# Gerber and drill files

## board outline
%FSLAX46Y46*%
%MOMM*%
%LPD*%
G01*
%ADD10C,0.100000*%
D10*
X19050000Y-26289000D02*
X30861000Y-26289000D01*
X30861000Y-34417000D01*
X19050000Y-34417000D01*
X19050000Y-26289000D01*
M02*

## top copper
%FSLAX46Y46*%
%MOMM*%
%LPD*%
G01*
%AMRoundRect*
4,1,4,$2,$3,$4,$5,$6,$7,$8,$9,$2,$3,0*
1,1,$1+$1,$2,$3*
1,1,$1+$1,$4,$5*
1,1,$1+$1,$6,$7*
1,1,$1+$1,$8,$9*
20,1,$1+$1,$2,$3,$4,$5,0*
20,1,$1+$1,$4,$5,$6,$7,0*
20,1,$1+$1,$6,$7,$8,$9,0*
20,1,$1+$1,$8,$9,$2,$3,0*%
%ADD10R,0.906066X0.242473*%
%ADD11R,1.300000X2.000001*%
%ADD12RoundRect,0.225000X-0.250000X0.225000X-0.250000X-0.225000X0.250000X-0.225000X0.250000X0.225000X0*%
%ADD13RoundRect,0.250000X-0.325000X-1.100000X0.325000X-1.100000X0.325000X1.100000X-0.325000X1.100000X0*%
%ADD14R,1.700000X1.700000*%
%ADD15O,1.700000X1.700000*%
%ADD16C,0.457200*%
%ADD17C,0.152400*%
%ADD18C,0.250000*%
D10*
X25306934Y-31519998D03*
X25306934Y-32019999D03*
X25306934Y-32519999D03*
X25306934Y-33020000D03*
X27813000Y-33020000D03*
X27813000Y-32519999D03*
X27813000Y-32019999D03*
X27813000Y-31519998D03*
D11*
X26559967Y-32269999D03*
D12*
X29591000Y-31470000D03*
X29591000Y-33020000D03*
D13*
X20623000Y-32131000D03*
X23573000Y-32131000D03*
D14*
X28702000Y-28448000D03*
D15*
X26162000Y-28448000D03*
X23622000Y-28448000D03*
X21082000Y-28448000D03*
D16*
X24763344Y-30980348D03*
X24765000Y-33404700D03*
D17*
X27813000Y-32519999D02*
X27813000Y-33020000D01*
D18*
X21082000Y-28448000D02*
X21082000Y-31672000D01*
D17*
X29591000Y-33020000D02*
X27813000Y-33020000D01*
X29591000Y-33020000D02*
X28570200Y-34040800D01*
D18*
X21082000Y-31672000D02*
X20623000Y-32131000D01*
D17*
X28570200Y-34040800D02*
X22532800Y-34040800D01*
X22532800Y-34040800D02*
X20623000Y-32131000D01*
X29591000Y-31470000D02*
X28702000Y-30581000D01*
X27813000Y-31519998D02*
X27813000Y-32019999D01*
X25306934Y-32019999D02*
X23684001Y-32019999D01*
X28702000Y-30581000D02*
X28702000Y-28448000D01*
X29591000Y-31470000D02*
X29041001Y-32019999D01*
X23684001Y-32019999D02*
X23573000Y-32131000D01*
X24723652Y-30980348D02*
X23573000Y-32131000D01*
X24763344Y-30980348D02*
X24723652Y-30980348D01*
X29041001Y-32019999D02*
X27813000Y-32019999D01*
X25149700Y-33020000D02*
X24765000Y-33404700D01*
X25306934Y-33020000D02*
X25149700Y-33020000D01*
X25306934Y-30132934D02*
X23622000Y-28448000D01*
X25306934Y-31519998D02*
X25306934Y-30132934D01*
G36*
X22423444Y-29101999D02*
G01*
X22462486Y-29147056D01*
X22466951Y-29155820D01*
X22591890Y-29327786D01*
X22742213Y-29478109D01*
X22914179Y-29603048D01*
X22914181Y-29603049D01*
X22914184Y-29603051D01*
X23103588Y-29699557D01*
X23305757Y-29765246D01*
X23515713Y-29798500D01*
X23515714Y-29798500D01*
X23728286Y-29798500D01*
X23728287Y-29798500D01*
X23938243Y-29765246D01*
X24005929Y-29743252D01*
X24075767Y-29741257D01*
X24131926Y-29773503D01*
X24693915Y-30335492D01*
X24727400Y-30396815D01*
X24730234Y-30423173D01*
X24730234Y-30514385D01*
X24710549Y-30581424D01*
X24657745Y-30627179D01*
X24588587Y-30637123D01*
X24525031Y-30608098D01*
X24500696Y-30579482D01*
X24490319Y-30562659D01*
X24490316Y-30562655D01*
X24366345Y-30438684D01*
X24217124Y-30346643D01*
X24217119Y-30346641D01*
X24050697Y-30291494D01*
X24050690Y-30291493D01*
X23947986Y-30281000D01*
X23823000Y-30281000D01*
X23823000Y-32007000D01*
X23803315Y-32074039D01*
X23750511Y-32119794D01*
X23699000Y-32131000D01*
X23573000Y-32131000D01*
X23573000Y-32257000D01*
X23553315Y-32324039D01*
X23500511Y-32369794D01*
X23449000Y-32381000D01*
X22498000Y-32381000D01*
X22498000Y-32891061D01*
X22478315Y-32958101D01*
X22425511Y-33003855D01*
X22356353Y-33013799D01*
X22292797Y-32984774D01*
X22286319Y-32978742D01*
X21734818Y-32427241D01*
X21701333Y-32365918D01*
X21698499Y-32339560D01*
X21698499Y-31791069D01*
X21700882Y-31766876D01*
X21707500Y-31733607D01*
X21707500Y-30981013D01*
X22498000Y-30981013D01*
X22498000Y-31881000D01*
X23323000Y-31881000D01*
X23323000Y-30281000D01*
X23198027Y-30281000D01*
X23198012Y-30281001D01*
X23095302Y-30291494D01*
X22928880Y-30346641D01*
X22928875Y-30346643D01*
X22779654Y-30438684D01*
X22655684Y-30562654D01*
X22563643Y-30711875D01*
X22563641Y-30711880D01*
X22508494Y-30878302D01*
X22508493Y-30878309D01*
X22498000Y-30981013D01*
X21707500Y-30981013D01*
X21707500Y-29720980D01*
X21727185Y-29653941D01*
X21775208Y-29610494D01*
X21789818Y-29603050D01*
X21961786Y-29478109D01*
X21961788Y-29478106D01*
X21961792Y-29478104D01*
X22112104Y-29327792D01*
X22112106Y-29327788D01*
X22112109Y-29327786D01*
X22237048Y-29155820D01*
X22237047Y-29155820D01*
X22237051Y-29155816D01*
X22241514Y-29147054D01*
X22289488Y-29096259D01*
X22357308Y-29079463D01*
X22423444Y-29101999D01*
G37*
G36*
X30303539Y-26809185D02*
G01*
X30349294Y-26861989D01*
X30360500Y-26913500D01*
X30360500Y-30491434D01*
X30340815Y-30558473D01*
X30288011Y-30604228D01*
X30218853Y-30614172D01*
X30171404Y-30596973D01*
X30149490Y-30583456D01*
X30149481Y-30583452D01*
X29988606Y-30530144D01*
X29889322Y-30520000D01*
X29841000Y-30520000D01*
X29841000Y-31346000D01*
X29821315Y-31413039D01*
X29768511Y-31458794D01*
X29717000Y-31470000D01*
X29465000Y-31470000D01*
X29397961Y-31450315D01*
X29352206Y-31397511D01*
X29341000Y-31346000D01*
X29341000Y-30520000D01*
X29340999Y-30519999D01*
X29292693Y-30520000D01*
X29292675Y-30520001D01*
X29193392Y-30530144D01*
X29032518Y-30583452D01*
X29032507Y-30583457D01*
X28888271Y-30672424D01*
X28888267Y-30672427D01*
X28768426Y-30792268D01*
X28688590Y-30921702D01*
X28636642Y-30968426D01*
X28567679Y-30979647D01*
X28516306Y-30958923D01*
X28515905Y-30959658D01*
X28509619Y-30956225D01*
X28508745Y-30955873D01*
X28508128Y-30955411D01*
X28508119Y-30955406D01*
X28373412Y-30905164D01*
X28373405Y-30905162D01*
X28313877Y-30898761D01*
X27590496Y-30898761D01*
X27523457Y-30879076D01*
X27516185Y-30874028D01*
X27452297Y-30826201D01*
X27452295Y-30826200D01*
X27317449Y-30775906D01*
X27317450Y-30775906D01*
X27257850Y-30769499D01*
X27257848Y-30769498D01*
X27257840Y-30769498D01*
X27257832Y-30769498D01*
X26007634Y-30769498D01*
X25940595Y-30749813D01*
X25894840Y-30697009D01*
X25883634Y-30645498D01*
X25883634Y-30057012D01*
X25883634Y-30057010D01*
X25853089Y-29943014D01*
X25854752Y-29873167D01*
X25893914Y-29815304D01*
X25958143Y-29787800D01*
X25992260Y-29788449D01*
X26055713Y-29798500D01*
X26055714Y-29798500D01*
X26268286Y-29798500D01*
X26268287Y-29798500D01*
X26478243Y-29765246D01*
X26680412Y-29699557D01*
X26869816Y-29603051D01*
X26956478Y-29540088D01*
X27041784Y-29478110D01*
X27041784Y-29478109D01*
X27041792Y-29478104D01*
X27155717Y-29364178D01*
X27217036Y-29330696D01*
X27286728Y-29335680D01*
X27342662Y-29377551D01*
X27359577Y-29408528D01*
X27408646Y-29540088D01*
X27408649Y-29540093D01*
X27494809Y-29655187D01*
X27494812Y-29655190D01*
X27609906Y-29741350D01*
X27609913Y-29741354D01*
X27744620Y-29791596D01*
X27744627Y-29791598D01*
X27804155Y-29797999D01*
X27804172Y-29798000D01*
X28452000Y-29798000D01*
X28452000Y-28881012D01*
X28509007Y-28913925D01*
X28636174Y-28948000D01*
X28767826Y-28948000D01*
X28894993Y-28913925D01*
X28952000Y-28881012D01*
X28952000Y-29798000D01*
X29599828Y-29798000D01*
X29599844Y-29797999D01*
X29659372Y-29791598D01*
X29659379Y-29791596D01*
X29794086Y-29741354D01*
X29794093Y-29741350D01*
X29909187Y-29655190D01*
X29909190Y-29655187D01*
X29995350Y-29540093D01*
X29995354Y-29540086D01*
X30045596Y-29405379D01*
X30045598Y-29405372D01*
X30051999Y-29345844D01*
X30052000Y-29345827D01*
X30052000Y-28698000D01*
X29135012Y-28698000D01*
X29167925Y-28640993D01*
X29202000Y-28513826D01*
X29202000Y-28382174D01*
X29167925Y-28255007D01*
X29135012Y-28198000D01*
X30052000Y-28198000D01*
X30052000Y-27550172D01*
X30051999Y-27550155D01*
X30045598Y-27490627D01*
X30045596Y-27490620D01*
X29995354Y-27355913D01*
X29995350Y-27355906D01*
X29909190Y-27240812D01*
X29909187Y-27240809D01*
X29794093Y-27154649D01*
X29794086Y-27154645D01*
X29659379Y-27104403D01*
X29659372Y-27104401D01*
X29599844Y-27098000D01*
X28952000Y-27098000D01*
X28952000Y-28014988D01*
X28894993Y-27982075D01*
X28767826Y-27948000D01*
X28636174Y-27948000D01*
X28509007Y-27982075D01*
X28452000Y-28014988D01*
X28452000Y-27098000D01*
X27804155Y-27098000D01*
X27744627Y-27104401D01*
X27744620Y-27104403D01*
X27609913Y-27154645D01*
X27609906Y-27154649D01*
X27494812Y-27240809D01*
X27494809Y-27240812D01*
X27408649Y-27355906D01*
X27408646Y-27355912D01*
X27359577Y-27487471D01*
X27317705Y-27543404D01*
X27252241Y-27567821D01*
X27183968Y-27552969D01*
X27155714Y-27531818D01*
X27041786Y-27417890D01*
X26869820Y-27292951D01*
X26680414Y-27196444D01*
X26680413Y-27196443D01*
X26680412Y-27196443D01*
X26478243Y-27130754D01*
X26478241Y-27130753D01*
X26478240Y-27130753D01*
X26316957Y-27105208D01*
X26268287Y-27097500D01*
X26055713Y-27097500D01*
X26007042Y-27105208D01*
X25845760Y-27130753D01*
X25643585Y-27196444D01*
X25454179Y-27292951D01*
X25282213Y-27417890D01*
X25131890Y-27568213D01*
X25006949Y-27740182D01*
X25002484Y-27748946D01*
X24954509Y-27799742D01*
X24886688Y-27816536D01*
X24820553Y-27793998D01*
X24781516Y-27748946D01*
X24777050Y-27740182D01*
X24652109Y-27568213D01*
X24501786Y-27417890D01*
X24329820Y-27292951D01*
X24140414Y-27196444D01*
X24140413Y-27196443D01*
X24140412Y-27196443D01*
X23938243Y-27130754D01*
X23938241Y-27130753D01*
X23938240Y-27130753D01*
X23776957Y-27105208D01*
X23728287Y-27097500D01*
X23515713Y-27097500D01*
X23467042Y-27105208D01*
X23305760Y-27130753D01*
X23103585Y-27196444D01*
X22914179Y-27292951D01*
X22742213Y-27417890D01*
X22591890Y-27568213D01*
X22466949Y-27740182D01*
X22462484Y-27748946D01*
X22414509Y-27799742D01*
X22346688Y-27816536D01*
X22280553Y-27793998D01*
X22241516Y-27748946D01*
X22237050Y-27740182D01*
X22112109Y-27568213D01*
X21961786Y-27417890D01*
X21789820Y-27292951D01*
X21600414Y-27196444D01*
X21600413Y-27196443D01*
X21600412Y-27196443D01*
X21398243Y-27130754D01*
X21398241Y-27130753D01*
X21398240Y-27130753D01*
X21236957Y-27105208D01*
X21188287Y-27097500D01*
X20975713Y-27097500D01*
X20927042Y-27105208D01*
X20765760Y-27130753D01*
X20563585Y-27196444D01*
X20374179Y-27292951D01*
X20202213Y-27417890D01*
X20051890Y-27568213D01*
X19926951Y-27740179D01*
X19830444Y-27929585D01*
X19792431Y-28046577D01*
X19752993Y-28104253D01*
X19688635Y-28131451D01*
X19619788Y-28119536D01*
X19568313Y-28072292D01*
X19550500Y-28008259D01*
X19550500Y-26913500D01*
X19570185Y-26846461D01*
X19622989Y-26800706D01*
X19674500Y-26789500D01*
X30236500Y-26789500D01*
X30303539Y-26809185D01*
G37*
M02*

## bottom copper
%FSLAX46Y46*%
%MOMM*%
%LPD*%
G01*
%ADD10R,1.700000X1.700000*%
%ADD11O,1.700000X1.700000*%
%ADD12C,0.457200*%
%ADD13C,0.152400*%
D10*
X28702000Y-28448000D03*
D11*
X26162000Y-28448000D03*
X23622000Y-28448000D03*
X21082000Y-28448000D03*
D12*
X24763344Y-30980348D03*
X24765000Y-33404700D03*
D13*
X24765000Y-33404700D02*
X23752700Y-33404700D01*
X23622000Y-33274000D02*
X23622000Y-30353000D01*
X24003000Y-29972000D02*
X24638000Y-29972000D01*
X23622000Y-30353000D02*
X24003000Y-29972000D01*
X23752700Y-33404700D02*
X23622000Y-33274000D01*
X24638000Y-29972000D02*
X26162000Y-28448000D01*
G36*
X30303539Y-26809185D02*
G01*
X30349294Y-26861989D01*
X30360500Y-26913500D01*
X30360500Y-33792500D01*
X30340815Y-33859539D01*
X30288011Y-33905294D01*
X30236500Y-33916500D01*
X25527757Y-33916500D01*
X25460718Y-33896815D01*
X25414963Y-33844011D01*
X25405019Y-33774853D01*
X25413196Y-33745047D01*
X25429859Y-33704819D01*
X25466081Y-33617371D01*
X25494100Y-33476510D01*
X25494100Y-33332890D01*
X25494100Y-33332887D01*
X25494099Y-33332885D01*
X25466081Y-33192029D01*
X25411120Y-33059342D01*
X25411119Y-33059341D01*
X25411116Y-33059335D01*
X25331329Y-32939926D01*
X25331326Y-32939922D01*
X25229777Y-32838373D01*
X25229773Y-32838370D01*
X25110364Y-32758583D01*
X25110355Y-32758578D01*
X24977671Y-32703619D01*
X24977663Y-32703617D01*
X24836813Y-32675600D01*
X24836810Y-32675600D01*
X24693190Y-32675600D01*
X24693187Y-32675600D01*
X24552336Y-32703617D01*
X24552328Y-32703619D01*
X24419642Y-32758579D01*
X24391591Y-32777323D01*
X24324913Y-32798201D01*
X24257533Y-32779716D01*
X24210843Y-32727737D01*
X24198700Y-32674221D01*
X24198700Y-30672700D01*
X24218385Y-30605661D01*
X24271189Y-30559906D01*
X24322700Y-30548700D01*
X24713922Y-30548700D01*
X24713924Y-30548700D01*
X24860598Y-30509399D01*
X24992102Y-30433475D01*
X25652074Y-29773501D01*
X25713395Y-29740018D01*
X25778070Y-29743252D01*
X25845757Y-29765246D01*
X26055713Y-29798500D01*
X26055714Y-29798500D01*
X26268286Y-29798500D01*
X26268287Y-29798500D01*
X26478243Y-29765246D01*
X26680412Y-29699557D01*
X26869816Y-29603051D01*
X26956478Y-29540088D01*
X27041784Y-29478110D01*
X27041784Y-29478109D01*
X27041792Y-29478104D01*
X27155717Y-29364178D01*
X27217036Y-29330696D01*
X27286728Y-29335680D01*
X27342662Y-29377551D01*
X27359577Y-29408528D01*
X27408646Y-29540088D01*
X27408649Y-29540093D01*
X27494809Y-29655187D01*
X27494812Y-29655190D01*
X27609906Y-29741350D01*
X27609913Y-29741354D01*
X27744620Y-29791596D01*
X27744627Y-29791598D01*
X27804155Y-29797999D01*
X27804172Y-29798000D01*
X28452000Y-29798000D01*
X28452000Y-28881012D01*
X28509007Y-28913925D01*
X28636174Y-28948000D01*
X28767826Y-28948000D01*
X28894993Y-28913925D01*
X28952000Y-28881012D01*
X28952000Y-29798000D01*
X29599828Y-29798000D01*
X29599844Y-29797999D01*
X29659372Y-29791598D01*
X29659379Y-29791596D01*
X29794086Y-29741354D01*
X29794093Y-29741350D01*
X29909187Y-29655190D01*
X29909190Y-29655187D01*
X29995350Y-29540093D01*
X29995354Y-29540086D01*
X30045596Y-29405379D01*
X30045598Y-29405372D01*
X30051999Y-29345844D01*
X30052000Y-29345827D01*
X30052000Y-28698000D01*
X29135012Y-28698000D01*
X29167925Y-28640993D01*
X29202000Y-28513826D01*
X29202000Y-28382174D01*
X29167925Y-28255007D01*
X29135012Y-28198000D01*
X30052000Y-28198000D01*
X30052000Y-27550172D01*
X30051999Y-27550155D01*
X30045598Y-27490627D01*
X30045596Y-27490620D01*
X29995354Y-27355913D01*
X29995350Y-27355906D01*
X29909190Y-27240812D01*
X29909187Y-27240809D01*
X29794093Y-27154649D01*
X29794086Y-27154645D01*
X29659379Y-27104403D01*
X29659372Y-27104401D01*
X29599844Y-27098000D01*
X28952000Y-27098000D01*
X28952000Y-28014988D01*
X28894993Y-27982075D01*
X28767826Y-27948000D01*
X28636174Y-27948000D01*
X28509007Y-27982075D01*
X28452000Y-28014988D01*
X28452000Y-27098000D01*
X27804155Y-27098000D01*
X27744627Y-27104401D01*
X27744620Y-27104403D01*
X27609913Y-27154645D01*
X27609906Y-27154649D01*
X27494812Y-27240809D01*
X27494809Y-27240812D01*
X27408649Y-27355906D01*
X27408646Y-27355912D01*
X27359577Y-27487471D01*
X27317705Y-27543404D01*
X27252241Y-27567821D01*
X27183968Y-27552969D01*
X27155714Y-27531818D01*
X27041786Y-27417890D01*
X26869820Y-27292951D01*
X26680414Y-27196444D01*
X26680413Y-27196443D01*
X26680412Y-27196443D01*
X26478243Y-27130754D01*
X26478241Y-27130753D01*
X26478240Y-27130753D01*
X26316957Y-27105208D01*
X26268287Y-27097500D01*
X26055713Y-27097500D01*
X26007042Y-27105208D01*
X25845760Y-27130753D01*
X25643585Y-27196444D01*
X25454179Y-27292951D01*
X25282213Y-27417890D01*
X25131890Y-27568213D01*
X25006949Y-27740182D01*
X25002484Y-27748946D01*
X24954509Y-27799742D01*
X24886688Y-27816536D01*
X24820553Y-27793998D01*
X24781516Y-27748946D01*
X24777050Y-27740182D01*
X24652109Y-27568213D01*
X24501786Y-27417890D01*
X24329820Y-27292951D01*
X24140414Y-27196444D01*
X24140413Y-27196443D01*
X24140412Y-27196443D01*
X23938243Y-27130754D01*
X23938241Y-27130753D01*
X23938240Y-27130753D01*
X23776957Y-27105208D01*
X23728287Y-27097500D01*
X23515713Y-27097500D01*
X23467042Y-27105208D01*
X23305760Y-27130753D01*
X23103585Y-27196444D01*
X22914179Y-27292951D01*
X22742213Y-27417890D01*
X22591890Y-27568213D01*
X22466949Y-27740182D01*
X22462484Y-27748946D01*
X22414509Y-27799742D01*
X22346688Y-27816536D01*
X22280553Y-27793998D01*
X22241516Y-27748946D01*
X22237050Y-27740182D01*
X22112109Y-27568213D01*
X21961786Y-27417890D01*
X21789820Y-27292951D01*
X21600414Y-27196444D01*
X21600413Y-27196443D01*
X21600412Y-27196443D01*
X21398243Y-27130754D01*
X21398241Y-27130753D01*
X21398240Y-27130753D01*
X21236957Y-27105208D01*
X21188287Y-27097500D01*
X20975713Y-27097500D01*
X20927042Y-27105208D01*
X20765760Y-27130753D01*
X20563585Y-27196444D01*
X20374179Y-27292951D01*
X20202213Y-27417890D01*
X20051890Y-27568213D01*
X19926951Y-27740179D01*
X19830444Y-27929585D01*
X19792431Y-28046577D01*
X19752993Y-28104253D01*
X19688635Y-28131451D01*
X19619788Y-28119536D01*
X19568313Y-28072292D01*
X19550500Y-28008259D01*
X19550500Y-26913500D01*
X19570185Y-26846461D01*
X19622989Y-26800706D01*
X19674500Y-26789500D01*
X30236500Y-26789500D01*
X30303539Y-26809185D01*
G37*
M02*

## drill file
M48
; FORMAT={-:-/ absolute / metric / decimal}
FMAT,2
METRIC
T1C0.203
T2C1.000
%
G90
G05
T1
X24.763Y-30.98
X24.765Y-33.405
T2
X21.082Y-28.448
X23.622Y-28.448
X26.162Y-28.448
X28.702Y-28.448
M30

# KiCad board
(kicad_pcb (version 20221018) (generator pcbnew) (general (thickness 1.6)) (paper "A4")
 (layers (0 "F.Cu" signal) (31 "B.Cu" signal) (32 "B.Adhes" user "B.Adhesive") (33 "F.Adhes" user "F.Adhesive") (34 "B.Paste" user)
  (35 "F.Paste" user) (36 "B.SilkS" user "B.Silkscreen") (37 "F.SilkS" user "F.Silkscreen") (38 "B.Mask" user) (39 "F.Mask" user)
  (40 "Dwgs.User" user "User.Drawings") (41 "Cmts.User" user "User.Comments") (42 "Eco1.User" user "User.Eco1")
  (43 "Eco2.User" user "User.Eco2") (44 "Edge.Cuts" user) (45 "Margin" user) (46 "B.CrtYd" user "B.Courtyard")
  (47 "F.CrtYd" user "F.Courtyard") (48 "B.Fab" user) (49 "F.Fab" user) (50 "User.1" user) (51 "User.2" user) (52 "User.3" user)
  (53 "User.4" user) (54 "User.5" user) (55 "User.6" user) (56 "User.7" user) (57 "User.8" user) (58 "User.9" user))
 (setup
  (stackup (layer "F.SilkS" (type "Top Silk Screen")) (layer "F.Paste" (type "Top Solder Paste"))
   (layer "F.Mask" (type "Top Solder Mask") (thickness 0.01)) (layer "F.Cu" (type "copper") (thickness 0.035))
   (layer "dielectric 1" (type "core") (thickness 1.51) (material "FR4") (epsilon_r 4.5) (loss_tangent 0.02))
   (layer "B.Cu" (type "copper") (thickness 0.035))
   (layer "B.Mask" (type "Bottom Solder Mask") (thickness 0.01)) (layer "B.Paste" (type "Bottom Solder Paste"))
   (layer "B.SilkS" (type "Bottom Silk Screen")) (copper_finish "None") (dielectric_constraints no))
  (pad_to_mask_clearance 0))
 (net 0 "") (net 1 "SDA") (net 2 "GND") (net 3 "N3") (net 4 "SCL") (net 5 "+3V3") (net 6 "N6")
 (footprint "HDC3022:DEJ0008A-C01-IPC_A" (layer "F.Cu") (at 26.559967 32.269999)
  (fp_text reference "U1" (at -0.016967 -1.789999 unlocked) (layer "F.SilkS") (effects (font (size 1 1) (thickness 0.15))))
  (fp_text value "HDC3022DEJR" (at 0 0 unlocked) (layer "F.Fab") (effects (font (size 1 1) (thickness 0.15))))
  (pad "1" smd rect (at -1.253033 -0.750001) (size 0.906066 0.242473) (layers "F.Cu" "F.Paste" "F.Mask") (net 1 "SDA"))
  (pad "2" smd rect (at -1.253033 -0.25) (size 0.906066 0.242473) (layers "F.Cu" "F.Paste" "F.Mask") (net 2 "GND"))
  (pad "3" smd rect (at -1.253033 0.25) (size 0.906066 0.242473) (layers "F.Cu" "F.Paste" "F.Mask") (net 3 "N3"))
  (pad "4" smd rect (at -1.253033 0.750001) (size 0.906066 0.242473) (layers "F.Cu" "F.Paste" "F.Mask") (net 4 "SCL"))
  (pad "5" smd rect (at 1.253033 0.750001) (size 0.906066 0.242473) (layers "F.Cu" "F.Paste" "F.Mask") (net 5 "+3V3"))
  (pad "6" smd rect (at 1.253033 0.25) (size 0.906066 0.242473) (layers "F.Cu" "F.Paste" "F.Mask") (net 5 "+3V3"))
  (pad "7" smd rect (at 1.253033 -0.25) (size 0.906066 0.242473) (layers "F.Cu" "F.Paste" "F.Mask") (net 2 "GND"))
  (pad "8" smd rect (at 1.253033 -0.750001) (size 0.906066 0.242473) (layers "F.Cu" "F.Paste" "F.Mask") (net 2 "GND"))
  (pad "9" smd rect (at 0 0) (size 1.3 2.000001) (layers "F.Cu" "F.Mask") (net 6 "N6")))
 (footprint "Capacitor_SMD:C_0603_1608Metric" (layer "F.Cu") (at 29.591 32.245 -90)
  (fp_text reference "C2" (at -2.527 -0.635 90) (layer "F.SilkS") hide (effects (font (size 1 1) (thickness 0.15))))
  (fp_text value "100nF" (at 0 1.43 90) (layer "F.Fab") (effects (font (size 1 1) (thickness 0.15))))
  (pad "1" smd roundrect (at -0.775 0 270) (size 0.9 0.95) (layers "F.Cu" "F.Paste" "F.Mask") (roundrect_rratio 0.25) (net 2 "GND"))
  (pad "2" smd roundrect (at 0.775 0 270) (size 0.9 0.95) (layers "F.Cu" "F.Paste" "F.Mask") (roundrect_rratio 0.25) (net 5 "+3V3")))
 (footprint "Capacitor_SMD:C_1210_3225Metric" (layer "F.Cu") (at 22.098 32.131)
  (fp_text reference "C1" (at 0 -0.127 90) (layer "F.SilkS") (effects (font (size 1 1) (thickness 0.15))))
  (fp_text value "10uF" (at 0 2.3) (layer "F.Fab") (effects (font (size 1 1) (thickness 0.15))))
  (pad "1" smd roundrect (at -1.475 0) (size 1.15 2.7) (layers "F.Cu" "F.Paste" "F.Mask") (roundrect_rratio 0.2173913043) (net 5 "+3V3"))
  (pad "2" smd roundrect (at 1.475 0) (size 1.15 2.7) (layers "F.Cu" "F.Paste" "F.Mask") (roundrect_rratio 0.2173913043) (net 2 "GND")))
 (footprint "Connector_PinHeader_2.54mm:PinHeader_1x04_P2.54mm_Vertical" (layer "F.Cu") (at 28.702 28.448 -90)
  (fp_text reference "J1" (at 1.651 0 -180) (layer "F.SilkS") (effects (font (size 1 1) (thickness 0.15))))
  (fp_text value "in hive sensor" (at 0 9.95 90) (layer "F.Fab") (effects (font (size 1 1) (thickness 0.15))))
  (pad "1" thru_hole rect (at 0 0 270) (size 1.7 1.7) (drill 1) (layers "*.Cu" "*.Mask") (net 2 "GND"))
  (pad "2" thru_hole oval (at 0 2.54 270) (size 1.7 1.7) (drill 1) (layers "*.Cu" "*.Mask") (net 4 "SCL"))
  (pad "3" thru_hole oval (at 0 5.08 270) (size 1.7 1.7) (drill 1) (layers "*.Cu" "*.Mask") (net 1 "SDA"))
  (pad "4" thru_hole oval (at 0 7.62 270) (size 1.7 1.7) (drill 1) (layers "*.Cu" "*.Mask") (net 5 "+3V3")))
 (gr_rect (start 19.05 26.289) (end 30.861 34.417) (stroke (width 0.1) (type default)) (fill none) (layer "Edge.Cuts"))
 (segment (start 27.813 32.519999) (end 27.813 33.02) (width 0.1524) (layer "F.Cu") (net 5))
 (segment (start 21.082 28.448) (end 21.082 31.672) (width 0.25) (layer "F.Cu") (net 5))
 (segment (start 29.591 33.02) (end 27.813 33.02) (width 0.1524) (layer "F.Cu") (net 5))
 (segment (start 29.591 33.02) (end 28.5702 34.0408) (width 0.1524) (layer "F.Cu") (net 5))
 (segment (start 21.082 31.672) (end 20.623 32.131) (width 0.25) (layer "F.Cu") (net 5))
 (segment (start 28.5702 34.0408) (end 22.5328 34.0408) (width 0.1524) (layer "F.Cu") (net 5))
 (segment (start 22.5328 34.0408) (end 20.623 32.131) (width 0.1524) (layer "F.Cu") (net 5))
 (segment (start 29.591 31.47) (end 28.702 30.581) (width 0.1524) (layer "F.Cu") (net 2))
 (segment (start 27.813 31.519998) (end 27.813 32.019999) (width 0.1524) (layer "F.Cu") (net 2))
 (segment (start 25.306934 32.019999) (end 23.684001 32.019999) (width 0.1524) (layer "F.Cu") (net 2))
 (segment (start 28.702 30.581) (end 28.702 28.448) (width 0.1524) (layer "F.Cu") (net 2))
 (segment (start 29.591 31.47) (end 29.041001 32.019999) (width 0.1524) (layer "F.Cu") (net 2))
 (segment (start 23.684001 32.019999) (end 23.573 32.131) (width 0.1524) (layer "F.Cu") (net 2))
 (segment (start 24.723652 30.980348) (end 23.573 32.131) (width 0.1524) (layer "F.Cu") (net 2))
 (segment (start 24.763344 30.980348) (end 24.723652 30.980348) (width 0.1524) (layer "F.Cu") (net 2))
 (segment (start 29.041001 32.019999) (end 27.813 32.019999) (width 0.1524) (layer "F.Cu") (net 2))
 (via (at 24.763344 30.980348) (size 0.4572) (drill 0.2032) (layers "F.Cu" "B.Cu") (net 2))
 (segment (start 25.1497 33.02) (end 24.765 33.4047) (width 0.1524) (layer "F.Cu") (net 4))
 (segment (start 25.306934 33.02) (end 25.1497 33.02) (width 0.1524) (layer "F.Cu") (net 4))
 (via (at 24.765 33.4047) (size 0.4572) (drill 0.2032) (layers "F.Cu" "B.Cu") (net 4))
 (segment (start 24.765 33.4047) (end 23.7527 33.4047) (width 0.1524) (layer "B.Cu") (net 4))
 (segment (start 23.622 33.274) (end 23.622 30.353) (width 0.1524) (layer "B.Cu") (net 4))
 (segment (start 24.003 29.972) (end 24.638 29.972) (width 0.1524) (layer "B.Cu") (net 4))
 (segment (start 23.622 30.353) (end 24.003 29.972) (width 0.1524) (layer "B.Cu") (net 4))
 (segment (start 23.7527 33.4047) (end 23.622 33.274) (width 0.1524) (layer "B.Cu") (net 4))
 (segment (start 24.638 29.972) (end 26.162 28.448) (width 0.1524) (layer "B.Cu") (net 4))
 (segment (start 25.306934 30.132934) (end 23.622 28.448) (width 0.1524) (layer "F.Cu") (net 1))
 (segment (start 25.306934 31.519998) (end 25.306934 30.132934) (width 0.1524) (layer "F.Cu") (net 1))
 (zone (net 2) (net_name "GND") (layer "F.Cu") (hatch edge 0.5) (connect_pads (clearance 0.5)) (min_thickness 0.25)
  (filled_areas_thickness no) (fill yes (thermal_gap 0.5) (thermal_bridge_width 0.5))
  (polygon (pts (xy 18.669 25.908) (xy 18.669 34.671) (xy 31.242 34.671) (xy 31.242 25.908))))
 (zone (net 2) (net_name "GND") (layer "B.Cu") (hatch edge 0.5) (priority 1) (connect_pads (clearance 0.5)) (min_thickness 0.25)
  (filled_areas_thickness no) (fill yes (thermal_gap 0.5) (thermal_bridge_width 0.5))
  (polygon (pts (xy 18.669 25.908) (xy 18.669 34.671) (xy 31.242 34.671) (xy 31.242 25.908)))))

